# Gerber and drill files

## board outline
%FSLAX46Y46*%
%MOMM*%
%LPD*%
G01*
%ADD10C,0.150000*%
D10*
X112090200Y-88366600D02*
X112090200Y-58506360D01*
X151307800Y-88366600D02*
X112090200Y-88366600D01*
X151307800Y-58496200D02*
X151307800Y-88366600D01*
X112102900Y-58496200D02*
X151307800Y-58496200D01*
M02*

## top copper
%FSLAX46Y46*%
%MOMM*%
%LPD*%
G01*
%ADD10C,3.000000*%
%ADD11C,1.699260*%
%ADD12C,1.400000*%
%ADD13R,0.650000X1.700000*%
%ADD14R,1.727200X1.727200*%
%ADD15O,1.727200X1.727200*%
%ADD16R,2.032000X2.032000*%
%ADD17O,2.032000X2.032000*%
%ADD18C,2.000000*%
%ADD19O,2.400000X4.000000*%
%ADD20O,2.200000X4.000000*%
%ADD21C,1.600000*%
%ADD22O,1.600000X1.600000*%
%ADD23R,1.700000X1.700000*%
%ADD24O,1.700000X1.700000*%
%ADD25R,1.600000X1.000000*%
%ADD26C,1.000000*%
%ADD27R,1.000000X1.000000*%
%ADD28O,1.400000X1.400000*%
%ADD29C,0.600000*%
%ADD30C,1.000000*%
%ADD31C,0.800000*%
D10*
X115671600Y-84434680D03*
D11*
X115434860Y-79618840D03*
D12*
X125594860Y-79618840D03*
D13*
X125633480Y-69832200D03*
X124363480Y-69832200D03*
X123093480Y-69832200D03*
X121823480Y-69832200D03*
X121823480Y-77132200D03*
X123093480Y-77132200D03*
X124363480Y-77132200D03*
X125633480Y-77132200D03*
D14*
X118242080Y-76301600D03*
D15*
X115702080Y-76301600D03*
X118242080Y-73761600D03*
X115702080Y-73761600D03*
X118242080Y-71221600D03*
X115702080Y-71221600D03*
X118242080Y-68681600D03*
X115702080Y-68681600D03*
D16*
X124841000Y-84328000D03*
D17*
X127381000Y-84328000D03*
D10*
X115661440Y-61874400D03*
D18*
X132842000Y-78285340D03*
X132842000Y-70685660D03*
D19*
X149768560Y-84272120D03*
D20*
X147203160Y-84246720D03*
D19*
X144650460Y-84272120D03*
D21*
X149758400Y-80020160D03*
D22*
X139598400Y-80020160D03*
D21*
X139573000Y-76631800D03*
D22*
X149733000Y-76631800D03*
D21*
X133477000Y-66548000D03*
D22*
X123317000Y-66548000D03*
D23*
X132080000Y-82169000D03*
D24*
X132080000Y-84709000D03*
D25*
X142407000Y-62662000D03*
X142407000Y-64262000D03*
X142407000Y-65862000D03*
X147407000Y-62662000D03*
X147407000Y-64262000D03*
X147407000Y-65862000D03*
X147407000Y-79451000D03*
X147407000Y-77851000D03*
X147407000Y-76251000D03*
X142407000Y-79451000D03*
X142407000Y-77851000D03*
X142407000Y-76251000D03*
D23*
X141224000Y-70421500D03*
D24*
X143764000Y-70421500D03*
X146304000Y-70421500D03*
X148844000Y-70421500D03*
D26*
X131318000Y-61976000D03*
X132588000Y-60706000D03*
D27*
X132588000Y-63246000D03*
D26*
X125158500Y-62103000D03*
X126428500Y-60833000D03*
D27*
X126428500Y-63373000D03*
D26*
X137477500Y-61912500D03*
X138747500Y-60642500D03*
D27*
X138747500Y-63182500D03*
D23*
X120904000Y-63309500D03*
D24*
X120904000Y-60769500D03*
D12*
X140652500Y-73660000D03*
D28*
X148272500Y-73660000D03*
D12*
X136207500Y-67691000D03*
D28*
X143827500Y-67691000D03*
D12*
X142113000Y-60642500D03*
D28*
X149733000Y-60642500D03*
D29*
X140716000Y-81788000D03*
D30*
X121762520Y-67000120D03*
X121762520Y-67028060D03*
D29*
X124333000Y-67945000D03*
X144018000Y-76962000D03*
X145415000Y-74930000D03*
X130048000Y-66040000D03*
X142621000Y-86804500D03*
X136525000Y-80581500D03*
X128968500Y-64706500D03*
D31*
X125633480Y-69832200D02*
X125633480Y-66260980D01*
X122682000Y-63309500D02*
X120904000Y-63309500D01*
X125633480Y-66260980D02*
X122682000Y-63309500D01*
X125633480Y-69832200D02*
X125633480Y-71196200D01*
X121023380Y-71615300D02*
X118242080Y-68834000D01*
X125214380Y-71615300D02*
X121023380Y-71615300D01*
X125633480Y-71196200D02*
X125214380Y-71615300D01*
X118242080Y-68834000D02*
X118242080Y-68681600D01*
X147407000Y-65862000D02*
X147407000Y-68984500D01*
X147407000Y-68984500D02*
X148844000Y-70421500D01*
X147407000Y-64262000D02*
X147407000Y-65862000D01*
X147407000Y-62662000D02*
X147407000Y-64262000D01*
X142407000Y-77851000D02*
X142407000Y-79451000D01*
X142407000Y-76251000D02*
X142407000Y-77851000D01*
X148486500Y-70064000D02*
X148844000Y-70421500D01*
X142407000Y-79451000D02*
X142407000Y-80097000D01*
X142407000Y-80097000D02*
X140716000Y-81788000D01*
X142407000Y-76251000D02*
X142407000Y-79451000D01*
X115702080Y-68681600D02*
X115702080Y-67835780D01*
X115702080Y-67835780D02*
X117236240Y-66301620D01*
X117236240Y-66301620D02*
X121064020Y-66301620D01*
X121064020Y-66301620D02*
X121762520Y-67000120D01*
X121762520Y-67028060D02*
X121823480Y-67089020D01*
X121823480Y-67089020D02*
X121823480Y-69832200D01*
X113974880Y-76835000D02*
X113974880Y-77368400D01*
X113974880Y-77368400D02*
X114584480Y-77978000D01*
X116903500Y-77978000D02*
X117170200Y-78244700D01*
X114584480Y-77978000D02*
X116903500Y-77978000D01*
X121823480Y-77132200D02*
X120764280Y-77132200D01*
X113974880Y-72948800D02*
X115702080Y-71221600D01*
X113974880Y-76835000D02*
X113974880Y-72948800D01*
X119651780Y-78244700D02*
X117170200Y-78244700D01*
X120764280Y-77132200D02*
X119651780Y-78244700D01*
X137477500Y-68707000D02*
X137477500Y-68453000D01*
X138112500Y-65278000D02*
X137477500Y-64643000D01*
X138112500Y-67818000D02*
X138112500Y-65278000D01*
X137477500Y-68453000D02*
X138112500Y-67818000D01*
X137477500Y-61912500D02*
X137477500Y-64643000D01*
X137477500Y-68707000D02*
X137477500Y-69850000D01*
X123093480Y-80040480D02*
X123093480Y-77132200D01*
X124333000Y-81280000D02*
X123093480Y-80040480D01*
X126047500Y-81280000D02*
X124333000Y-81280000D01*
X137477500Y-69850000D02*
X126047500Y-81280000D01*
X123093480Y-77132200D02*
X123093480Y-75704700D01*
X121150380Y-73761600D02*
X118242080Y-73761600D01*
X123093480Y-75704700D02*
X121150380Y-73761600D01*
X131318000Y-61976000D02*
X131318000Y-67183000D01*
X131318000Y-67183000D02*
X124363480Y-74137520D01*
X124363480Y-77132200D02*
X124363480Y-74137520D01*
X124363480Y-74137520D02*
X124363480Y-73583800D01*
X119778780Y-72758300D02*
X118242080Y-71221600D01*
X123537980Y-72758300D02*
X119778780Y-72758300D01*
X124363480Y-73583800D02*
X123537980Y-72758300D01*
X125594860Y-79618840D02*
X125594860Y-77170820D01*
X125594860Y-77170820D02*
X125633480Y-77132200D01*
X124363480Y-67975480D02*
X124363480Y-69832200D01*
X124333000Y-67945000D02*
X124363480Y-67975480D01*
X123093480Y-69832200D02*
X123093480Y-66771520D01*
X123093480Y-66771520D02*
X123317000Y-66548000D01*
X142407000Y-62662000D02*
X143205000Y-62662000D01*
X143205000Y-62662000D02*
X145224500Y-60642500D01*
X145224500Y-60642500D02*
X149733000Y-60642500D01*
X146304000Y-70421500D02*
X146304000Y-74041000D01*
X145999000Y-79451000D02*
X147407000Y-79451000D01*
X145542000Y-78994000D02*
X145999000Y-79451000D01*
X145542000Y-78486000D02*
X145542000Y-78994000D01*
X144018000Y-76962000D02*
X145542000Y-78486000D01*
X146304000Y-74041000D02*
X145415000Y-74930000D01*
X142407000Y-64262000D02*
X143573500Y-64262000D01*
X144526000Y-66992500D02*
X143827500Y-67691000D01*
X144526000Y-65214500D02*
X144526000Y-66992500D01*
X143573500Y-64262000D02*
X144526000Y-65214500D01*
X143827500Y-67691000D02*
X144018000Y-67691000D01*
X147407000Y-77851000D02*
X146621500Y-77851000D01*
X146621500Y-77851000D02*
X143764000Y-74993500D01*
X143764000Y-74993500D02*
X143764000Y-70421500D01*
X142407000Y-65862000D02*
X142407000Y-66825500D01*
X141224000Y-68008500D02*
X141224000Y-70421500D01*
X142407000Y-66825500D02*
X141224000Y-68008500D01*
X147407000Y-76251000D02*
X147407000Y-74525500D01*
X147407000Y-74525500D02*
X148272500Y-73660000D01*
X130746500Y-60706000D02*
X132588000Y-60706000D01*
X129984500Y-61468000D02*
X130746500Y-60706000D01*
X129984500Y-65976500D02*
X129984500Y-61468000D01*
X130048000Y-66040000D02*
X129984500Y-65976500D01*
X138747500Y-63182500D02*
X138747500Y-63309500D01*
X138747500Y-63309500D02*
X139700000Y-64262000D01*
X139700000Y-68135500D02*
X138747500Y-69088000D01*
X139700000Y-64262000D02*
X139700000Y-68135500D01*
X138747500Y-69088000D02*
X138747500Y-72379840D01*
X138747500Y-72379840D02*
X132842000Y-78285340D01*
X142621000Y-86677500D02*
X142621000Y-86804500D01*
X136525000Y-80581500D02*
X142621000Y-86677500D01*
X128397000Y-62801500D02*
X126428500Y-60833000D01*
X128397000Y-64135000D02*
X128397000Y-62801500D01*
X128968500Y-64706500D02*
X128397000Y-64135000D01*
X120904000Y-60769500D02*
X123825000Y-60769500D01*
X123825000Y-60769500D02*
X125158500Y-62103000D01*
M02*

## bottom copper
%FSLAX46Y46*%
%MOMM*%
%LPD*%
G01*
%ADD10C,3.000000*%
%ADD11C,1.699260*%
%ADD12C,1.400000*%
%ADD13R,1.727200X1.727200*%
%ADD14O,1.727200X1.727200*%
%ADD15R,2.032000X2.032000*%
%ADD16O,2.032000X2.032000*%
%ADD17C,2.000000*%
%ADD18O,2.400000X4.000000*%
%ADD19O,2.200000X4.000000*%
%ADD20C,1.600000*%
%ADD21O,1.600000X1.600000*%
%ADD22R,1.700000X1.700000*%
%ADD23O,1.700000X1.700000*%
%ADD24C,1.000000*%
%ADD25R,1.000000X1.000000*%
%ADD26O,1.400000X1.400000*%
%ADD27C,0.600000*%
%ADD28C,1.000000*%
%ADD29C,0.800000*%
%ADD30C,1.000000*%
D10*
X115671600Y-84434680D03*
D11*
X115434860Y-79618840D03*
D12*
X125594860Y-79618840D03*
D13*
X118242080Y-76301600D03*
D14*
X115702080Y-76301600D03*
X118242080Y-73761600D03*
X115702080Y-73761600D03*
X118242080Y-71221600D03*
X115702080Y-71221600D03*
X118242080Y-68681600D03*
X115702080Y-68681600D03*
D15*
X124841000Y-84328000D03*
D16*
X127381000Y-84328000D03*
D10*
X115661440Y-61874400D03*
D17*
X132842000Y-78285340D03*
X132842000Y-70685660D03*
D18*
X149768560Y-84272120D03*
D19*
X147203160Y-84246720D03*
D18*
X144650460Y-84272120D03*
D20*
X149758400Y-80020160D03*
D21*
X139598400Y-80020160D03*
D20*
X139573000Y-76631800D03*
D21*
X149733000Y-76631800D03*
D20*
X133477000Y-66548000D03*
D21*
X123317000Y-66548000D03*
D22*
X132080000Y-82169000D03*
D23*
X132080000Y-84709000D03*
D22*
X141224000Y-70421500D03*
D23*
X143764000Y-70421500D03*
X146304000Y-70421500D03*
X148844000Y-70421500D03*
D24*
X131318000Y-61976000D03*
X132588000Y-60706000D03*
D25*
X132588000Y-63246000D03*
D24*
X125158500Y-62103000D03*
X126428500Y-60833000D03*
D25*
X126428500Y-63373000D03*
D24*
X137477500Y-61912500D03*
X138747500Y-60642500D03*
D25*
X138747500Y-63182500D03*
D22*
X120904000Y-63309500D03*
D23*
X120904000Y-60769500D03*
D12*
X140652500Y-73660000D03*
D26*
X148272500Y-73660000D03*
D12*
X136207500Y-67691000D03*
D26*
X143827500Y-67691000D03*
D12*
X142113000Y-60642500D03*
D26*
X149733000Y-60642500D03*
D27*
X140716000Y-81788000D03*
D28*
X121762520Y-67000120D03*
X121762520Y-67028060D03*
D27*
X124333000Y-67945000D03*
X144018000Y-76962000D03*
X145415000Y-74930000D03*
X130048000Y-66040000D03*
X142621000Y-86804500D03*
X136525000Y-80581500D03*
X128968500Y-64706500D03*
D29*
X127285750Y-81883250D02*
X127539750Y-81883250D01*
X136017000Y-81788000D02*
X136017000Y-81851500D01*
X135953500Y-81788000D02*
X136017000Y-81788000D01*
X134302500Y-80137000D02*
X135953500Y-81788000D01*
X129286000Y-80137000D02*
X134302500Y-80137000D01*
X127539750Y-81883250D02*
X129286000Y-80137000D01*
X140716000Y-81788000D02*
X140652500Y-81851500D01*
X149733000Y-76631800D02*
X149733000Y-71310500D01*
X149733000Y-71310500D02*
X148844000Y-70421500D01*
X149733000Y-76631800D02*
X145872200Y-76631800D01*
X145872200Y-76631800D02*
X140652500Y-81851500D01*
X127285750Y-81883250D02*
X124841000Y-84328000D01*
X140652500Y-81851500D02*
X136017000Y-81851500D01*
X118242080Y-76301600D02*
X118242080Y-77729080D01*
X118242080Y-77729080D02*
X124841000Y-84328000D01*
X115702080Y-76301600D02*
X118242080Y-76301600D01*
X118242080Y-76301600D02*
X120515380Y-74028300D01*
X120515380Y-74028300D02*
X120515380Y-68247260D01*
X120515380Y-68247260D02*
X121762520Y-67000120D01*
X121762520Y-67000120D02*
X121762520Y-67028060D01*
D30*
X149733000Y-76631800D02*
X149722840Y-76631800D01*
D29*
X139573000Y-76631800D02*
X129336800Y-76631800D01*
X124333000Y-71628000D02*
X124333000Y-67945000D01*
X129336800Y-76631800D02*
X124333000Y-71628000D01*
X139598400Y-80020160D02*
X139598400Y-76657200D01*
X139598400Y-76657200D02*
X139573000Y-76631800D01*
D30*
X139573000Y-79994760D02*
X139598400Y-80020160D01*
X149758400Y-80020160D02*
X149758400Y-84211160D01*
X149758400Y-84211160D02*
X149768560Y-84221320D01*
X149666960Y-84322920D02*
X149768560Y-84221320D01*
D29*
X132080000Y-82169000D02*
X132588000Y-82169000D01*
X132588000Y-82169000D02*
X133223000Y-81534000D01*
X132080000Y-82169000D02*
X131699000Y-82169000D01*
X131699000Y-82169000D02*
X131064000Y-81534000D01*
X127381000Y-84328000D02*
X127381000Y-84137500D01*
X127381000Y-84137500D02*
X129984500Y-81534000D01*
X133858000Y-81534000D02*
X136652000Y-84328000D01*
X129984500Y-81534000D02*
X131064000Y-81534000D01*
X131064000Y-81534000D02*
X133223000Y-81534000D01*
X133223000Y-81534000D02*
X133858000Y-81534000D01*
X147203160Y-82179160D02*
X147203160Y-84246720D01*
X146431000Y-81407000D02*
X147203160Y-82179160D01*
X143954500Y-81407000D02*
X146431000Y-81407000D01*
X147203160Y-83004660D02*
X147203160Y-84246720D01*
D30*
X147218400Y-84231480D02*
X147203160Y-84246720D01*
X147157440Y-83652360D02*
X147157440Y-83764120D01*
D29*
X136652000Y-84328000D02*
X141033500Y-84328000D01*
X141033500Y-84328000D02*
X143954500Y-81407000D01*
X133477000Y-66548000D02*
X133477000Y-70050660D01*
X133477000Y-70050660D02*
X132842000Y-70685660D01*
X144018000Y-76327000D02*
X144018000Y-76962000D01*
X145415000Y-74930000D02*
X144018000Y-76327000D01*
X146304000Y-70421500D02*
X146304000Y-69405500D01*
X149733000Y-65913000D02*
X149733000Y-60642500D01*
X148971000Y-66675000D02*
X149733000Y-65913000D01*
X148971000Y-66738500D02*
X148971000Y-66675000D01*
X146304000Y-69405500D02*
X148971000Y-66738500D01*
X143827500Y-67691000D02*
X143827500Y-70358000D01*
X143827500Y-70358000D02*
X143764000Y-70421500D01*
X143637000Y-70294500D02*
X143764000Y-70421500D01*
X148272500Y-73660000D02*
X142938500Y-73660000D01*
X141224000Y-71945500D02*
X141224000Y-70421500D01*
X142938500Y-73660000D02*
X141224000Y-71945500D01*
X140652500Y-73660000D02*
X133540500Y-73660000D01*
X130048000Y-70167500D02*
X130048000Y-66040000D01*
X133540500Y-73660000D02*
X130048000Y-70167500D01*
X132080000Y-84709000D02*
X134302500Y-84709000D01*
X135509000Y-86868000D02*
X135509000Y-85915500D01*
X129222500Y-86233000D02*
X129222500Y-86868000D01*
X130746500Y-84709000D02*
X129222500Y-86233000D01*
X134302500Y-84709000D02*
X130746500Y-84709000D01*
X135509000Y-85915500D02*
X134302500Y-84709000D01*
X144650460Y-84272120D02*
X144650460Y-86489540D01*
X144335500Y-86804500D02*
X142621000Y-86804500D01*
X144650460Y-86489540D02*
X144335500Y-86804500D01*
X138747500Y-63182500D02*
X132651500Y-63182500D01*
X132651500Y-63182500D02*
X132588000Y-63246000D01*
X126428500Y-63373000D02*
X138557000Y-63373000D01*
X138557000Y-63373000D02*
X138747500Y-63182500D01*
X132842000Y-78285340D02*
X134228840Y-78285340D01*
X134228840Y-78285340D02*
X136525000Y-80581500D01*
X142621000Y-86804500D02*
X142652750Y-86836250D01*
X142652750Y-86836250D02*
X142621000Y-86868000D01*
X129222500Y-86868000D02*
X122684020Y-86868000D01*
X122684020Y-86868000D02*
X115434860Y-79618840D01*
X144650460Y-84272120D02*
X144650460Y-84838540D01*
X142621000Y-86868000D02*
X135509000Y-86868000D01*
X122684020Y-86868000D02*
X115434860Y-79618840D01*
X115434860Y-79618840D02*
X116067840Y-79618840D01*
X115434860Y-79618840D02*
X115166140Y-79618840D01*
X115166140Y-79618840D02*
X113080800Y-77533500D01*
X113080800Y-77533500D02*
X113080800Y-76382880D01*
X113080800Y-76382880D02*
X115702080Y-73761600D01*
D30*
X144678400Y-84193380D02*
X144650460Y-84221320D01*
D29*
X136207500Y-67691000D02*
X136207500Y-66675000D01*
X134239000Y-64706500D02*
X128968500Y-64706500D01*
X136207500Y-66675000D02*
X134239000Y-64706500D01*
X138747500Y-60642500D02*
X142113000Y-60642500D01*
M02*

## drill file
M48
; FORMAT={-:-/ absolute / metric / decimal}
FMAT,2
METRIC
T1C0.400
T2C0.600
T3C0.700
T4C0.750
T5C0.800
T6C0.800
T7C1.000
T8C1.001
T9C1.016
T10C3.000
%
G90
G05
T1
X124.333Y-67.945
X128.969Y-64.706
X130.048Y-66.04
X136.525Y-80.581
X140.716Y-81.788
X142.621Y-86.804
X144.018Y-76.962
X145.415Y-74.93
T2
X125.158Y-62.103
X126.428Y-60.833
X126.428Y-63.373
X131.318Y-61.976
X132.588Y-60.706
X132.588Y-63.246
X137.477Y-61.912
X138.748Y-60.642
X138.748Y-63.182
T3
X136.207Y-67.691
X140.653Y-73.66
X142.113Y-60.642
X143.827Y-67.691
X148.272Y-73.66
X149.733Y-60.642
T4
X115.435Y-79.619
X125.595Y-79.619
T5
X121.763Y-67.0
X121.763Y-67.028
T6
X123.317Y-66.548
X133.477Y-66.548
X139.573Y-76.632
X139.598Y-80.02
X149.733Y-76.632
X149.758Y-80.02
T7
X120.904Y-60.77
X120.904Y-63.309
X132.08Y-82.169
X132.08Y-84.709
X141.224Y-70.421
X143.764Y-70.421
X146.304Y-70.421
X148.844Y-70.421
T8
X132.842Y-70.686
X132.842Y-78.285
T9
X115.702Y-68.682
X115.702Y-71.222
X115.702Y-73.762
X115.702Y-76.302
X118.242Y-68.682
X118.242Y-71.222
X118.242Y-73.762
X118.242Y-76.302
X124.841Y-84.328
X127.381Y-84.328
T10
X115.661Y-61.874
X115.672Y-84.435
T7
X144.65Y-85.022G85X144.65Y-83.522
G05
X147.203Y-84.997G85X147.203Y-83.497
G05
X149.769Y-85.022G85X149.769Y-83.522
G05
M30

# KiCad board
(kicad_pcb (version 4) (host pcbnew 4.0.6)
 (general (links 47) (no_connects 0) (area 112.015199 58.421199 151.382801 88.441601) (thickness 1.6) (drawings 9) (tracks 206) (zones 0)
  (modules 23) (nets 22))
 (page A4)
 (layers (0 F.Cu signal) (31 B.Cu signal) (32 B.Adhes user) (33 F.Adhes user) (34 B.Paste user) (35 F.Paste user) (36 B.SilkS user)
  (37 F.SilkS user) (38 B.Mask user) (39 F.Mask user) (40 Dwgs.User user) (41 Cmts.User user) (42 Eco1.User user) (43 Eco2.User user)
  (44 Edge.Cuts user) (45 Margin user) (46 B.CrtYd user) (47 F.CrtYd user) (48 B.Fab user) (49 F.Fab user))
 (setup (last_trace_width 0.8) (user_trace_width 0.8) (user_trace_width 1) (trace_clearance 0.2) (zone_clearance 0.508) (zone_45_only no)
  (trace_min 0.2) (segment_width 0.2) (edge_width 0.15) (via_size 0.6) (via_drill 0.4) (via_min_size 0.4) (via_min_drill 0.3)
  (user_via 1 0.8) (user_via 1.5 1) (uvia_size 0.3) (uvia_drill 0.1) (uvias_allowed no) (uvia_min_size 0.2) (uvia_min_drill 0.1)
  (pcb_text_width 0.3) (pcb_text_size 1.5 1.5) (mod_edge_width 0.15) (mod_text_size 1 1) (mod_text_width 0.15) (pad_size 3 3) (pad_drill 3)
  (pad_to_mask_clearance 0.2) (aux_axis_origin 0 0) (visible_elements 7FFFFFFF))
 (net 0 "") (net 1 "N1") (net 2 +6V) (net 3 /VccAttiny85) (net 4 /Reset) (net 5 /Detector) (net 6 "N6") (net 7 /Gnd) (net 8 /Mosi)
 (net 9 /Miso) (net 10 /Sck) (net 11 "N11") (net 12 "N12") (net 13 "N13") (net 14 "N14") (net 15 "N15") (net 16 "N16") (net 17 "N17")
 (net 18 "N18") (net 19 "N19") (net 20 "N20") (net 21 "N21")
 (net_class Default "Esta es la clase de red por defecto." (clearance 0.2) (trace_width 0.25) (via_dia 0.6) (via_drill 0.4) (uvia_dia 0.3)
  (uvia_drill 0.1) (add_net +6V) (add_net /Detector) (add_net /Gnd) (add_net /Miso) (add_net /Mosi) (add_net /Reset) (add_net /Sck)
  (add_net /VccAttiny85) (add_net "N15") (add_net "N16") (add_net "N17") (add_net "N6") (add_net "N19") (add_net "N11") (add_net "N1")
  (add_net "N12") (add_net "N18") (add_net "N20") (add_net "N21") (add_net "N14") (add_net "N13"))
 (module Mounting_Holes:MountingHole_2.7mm (layer F.Cu) (at 115.6716 84.43468)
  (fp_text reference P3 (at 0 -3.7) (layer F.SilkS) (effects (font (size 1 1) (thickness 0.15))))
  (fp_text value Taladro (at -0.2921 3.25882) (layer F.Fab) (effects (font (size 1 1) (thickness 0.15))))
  (pad 1 thru_hole circle (at 0 0) (size 3 3) (drill 3) (layers *.Cu *.Mask) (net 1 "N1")))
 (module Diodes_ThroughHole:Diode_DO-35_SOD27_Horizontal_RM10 (layer F.Cu) (at 125.59538 79.6163 180)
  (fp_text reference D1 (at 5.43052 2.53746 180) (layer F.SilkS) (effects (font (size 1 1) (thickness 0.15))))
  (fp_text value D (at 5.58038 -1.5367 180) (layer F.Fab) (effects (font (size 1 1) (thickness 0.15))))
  (pad 2 thru_hole circle (at 10.16052 -0.00254) (size 1.69926 1.69926) (drill 0.75) (layers *.Cu *.Mask) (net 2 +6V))
  (pad 1 thru_hole circle (at 0.00052 -0.00254) (size 1.4 1.4) (drill 0.75) (layers *.Cu *.Mask) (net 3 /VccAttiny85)))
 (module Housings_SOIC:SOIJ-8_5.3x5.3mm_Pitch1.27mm (layer F.Cu) (at 123.72848 73.4822 270)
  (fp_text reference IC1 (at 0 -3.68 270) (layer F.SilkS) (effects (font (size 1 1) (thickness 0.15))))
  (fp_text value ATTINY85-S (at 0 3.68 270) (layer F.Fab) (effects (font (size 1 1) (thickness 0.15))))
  (pad 1 smd rect (at -3.65 -1.905 270) (size 1.7 0.65) (layers F.Cu F.Paste F.Mask) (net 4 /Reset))
  (pad 2 smd rect (at -3.65 -0.635 270) (size 1.7 0.65) (layers F.Cu F.Paste F.Mask) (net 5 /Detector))
  (pad 3 smd rect (at -3.65 0.635 270) (size 1.7 0.65) (layers F.Cu F.Paste F.Mask) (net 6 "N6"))
  (pad 4 smd rect (at -3.65 1.905 270) (size 1.7 0.65) (layers F.Cu F.Paste F.Mask) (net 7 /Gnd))
  (pad 5 smd rect (at 3.65 1.905 270) (size 1.7 0.65) (layers F.Cu F.Paste F.Mask) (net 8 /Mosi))
  (pad 6 smd rect (at 3.65 0.635 270) (size 1.7 0.65) (layers F.Cu F.Paste F.Mask) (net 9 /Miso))
  (pad 7 smd rect (at 3.65 -0.635 270) (size 1.7 0.65) (layers F.Cu F.Paste F.Mask) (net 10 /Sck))
  (pad 8 smd rect (at 3.65 -1.905 270) (size 1.7 0.65) (layers F.Cu F.Paste F.Mask) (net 3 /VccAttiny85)))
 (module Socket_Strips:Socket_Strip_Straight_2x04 (layer B.Cu) (at 118.24208 76.3016 90)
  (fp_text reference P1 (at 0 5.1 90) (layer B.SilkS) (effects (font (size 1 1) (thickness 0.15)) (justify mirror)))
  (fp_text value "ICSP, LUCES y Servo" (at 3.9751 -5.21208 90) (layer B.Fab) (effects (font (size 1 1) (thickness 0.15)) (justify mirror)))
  (pad 1 thru_hole rect (at 0 0 90) (size 1.7272 1.7272) (drill 1.016) (layers *.Cu *.Mask) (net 7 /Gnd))
  (pad 2 thru_hole oval (at 0 -2.54 90) (size 1.7272 1.7272) (drill 1.016) (layers *.Cu *.Mask) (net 7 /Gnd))
  (pad 3 thru_hole oval (at 2.54 0 90) (size 1.7272 1.7272) (drill 1.016) (layers *.Cu *.Mask) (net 9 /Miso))
  (pad 4 thru_hole oval (at 2.54 -2.54 90) (size 1.7272 1.7272) (drill 1.016) (layers *.Cu *.Mask) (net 2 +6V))
  (pad 5 thru_hole oval (at 5.08 0 90) (size 1.7272 1.7272) (drill 1.016) (layers *.Cu *.Mask) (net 10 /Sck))
  (pad 6 thru_hole oval (at 5.08 -2.54 90) (size 1.7272 1.7272) (drill 1.016) (layers *.Cu *.Mask) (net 8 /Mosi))
  (pad 7 thru_hole oval (at 7.62 0 90) (size 1.7272 1.7272) (drill 1.016) (layers *.Cu *.Mask) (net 4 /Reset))
  (pad 8 thru_hole oval (at 7.62 -2.54 90) (size 1.7272 1.7272) (drill 1.016) (layers *.Cu *.Mask) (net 7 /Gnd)))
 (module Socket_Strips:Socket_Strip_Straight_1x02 (layer F.Cu) (at 124.841 84.328)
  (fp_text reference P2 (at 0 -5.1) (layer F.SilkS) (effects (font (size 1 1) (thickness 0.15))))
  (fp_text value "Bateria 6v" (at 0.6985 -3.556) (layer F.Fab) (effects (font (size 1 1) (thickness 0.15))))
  (pad 1 thru_hole rect (at 0 0) (size 2.032 2.032) (drill 1.016) (layers *.Cu *.Mask) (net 7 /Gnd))
  (pad 2 thru_hole oval (at 2.54 0) (size 2.032 2.032) (drill 1.016) (layers *.Cu *.Mask) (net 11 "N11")))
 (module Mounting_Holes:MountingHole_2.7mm (layer F.Cu) (at 115.66144 61.8744)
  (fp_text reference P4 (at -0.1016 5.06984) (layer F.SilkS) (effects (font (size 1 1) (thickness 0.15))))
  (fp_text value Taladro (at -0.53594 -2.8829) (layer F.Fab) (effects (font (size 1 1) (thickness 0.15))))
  (pad 1 thru_hole circle (at 0 0) (size 3 3) (drill 3) (layers *.Cu *.Mask) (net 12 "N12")))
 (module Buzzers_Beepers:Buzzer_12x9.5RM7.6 (layer F.Cu) (at 132.842 74.4855 90)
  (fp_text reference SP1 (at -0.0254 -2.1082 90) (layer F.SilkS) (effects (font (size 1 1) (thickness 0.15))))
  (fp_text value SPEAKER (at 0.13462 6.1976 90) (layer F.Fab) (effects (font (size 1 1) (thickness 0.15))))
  (pad 1 thru_hole circle (at -3.79984 0 90) (size 2 2) (drill 1.00076) (layers *.Cu *.Mask) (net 2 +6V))
  (pad 2 thru_hole circle (at 3.79984 0 90) (size 2 2) (drill 1.00076) (layers *.Cu *.Mask) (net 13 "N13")))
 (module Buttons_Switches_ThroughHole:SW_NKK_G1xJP (layer B.Cu) (at 147.17776 84.24672 180)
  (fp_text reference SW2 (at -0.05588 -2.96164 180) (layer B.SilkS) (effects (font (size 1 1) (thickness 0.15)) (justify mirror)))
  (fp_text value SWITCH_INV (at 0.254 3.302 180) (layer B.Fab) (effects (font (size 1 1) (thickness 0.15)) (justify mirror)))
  (pad 1 thru_hole oval (at -2.5908 -0.0254 180) (size 2.4 4) (drill oval 1 2.5) (layers *.Cu *.Mask) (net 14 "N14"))
  (pad 2 thru_hole oval (at -0.0254 0 180) (size 2.2 4) (drill oval 1 2.5) (layers *.Cu *.Mask) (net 11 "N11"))
  (pad 3 thru_hole oval (at 2.5273 -0.0254 180) (size 2.4 4) (drill oval 1 2.5) (layers *.Cu *.Mask) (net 2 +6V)))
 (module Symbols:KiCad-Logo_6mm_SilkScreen (layer B.Cu) (at 132.6515 74.676)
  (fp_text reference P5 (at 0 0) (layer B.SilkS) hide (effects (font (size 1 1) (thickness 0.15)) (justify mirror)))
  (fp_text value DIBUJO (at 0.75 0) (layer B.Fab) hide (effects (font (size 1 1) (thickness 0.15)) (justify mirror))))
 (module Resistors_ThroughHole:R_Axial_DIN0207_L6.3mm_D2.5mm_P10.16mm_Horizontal (layer B.Cu) (at 149.7584 80.02016 180)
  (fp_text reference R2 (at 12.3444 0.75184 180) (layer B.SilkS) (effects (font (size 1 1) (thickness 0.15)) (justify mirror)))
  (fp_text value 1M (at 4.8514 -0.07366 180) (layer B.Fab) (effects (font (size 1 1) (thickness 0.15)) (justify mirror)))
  (pad 1 thru_hole circle (at 0 0 180) (size 1.6 1.6) (drill 0.8) (layers *.Cu *.Mask) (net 14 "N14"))
  (pad 2 thru_hole oval (at 10.16 0 180) (size 1.6 1.6) (drill 0.8) (layers *.Cu *.Mask) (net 5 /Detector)))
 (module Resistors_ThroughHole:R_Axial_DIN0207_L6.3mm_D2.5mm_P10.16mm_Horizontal (layer B.Cu) (at 139.573 76.6318)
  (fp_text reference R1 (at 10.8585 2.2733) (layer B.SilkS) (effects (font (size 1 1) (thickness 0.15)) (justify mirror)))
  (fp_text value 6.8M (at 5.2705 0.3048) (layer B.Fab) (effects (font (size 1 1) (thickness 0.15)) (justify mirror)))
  (pad 1 thru_hole circle (at 0 0) (size 1.6 1.6) (drill 0.8) (layers *.Cu *.Mask) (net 5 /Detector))
  (pad 2 thru_hole oval (at 10.16 0) (size 1.6 1.6) (drill 0.8) (layers *.Cu *.Mask) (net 7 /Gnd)))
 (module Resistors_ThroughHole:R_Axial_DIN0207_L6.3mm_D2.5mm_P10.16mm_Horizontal (layer F.Cu) (at 133.477 66.548 180)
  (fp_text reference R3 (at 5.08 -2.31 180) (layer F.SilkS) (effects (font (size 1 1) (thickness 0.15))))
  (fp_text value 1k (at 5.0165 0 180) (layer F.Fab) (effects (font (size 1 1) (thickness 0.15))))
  (pad 1 thru_hole circle (at 0 0 180) (size 1.6 1.6) (drill 0.8) (layers *.Cu *.Mask) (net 13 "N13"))
  (pad 2 thru_hole oval (at 10.16 0 180) (size 1.6 1.6) (drill 0.8) (layers *.Cu *.Mask) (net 6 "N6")))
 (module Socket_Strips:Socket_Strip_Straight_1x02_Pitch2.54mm (layer F.Cu) (at 132.08 82.169)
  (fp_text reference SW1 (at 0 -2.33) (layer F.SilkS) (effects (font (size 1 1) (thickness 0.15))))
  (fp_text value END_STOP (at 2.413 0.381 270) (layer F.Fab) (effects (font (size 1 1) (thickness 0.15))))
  (pad 1 thru_hole rect (at 0 0) (size 1.7 1.7) (drill 1) (layers *.Cu *.Mask) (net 11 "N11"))
  (pad 2 thru_hole oval (at 0 2.54) (size 1.7 1.7) (drill 1) (layers *.Cu *.Mask) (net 2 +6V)))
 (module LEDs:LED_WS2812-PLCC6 (layer F.Cu) (at 144.907 64.262 180)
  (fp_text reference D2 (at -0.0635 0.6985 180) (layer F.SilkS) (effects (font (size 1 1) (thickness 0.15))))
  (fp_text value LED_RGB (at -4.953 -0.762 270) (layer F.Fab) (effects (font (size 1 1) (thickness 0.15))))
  (pad 4 smd rect (at 2.5 1.6 180) (size 1.6 1) (layers F.Cu F.Paste F.Mask) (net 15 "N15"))
  (pad 5 smd rect (at 2.5 0 180) (size 1.6 1) (layers F.Cu F.Paste F.Mask) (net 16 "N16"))
  (pad 6 smd rect (at 2.5 -1.6 180) (size 1.6 1) (layers F.Cu F.Paste F.Mask) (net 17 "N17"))
  (pad 3 smd rect (at -2.5 1.6 180) (size 1.6 1) (layers F.Cu F.Paste F.Mask) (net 7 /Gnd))
  (pad 2 smd rect (at -2.5 0 180) (size 1.6 1) (layers F.Cu F.Paste F.Mask) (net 7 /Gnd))
  (pad 1 smd rect (at -2.5 -1.6 180) (size 1.6 1) (layers F.Cu F.Paste F.Mask) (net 7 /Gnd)))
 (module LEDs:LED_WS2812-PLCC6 (layer F.Cu) (at 144.907 77.851)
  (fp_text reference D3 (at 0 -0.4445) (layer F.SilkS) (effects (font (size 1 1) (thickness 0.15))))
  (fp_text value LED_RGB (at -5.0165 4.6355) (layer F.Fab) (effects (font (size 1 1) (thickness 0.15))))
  (pad 4 smd rect (at 2.5 1.6) (size 1.6 1) (layers F.Cu F.Paste F.Mask) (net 15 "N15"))
  (pad 5 smd rect (at 2.5 0) (size 1.6 1) (layers F.Cu F.Paste F.Mask) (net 16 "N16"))
  (pad 6 smd rect (at 2.5 -1.6) (size 1.6 1) (layers F.Cu F.Paste F.Mask) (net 17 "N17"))
  (pad 3 smd rect (at -2.5 1.6) (size 1.6 1) (layers F.Cu F.Paste F.Mask) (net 7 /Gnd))
  (pad 2 smd rect (at -2.5 0) (size 1.6 1) (layers F.Cu F.Paste F.Mask) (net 7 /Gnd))
  (pad 1 smd rect (at -2.5 -1.6) (size 1.6 1) (layers F.Cu F.Paste F.Mask) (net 7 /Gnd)))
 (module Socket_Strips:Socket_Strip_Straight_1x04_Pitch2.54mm (layer F.Cu) (at 141.224 70.4215 90)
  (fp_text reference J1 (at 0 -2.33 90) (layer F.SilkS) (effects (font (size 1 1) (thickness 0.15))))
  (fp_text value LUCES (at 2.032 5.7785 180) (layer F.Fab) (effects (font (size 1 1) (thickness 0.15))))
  (pad 1 thru_hole rect (at 0 0 90) (size 1.7 1.7) (drill 1) (layers *.Cu *.Mask) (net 17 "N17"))
  (pad 2 thru_hole oval (at 0 2.54 90) (size 1.7 1.7) (drill 1) (layers *.Cu *.Mask) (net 16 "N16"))
  (pad 3 thru_hole oval (at 0 5.08 90) (size 1.7 1.7) (drill 1) (layers *.Cu *.Mask) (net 15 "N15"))
  (pad 4 thru_hole oval (at 0 7.62 90) (size 1.7 1.7) (drill 1) (layers *.Cu *.Mask) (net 7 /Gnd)))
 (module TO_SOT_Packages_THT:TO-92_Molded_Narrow (layer F.Cu) (at 132.588 63.246 90)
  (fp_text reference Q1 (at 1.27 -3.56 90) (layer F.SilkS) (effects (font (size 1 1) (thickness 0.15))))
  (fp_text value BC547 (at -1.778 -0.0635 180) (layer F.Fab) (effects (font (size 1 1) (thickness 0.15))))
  (pad 2 thru_hole circle (at 1.27 -1.27 180) (size 1 1) (drill 0.6) (layers *.Cu *.Mask) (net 10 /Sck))
  (pad 3 thru_hole circle (at 2.54 0 180) (size 1 1) (drill 0.6) (layers *.Cu *.Mask) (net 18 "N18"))
  (pad 1 thru_hole rect (at 0 0 180) (size 1 1) (drill 0.6) (layers *.Cu *.Mask) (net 2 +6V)))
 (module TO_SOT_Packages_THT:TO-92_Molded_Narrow (layer F.Cu) (at 126.4285 63.373 90)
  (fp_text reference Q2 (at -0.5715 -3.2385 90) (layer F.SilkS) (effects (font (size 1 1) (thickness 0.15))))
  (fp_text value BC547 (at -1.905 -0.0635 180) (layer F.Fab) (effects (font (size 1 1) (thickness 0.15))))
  (pad 2 thru_hole circle (at 1.27 -1.27 180) (size 1 1) (drill 0.6) (layers *.Cu *.Mask) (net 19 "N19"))
  (pad 3 thru_hole circle (at 2.54 0 180) (size 1 1) (drill 0.6) (layers *.Cu *.Mask) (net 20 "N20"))
  (pad 1 thru_hole rect (at 0 0 180) (size 1 1) (drill 0.6) (layers *.Cu *.Mask) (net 2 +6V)))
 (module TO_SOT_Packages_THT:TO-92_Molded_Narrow (layer F.Cu) (at 138.7475 63.1825 90)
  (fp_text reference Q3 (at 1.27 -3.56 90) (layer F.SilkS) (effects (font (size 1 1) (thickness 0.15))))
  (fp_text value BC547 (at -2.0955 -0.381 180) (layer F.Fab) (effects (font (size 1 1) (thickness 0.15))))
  (pad 2 thru_hole circle (at 1.27 -1.27 180) (size 1 1) (drill 0.6) (layers *.Cu *.Mask) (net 9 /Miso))
  (pad 3 thru_hole circle (at 2.54 0 180) (size 1 1) (drill 0.6) (layers *.Cu *.Mask) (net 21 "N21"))
  (pad 1 thru_hole rect (at 0 0 180) (size 1 1) (drill 0.6) (layers *.Cu *.Mask) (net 2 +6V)))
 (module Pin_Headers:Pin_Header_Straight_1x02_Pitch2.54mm (layer F.Cu) (at 120.904 63.3095 180)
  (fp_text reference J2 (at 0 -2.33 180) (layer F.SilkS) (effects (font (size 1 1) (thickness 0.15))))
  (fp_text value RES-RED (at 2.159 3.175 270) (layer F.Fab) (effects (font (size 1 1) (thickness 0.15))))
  (pad 1 thru_hole rect (at 0 0 180) (size 1.7 1.7) (drill 1) (layers *.Cu *.Mask) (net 4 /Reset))
  (pad 2 thru_hole oval (at 0 2.54 180) (size 1.7 1.7) (drill 1) (layers *.Cu *.Mask) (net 19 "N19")))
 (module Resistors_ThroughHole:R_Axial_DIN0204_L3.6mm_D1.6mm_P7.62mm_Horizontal (layer F.Cu) (at 140.6525 73.66)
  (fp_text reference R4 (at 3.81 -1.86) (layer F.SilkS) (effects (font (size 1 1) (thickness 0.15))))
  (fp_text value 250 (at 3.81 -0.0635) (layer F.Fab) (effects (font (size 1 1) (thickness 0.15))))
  (pad 1 thru_hole circle (at 0 0) (size 1.4 1.4) (drill 0.7) (layers *.Cu *.Mask) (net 18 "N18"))
  (pad 2 thru_hole oval (at 7.62 0) (size 1.4 1.4) (drill 0.7) (layers *.Cu *.Mask) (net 17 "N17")))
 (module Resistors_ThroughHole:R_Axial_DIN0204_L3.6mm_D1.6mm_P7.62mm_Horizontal (layer F.Cu) (at 136.2075 67.691)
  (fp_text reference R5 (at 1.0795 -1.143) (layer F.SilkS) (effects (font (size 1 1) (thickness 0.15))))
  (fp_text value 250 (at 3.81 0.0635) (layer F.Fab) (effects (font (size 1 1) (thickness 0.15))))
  (pad 1 thru_hole circle (at 0 0) (size 1.4 1.4) (drill 0.7) (layers *.Cu *.Mask) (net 20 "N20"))
  (pad 2 thru_hole oval (at 7.62 0) (size 1.4 1.4) (drill 0.7) (layers *.Cu *.Mask) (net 16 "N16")))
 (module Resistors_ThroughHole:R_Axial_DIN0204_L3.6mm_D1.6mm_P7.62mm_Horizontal (layer F.Cu) (at 142.113 60.6425)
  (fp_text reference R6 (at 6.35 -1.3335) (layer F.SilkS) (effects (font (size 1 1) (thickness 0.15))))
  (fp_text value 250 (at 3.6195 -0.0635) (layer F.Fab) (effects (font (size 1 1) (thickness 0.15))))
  (pad 1 thru_hole circle (at 0 0) (size 1.4 1.4) (drill 0.7) (layers *.Cu *.Mask) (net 21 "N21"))
  (pad 2 thru_hole oval (at 7.62 0) (size 1.4 1.4) (drill 0.7) (layers *.Cu *.Mask) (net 15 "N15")))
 (gr_line (start 112.0902 88.3666) (end 112.0902 58.50636) (angle 90) (layer Edge.Cuts) (width 0.15))
 (gr_line (start 151.3078 88.3666) (end 112.0902 88.3666) (angle 90) (layer Edge.Cuts) (width 0.15))
 (gr_line (start 151.3078 58.4962) (end 151.3078 88.3666) (angle 90) (layer Edge.Cuts) (width 0.15))
 (gr_line (start 112.1029 58.4962) (end 151.3078 58.4962) (angle 90) (layer Edge.Cuts) (width 0.15))
 (segment (start 125.63348 69.8322) (end 125.63348 66.26098) (width 0.8) (layer F.Cu) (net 4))
 (segment (start 122.682 63.3095) (end 120.904 63.3095) (width 0.8) (layer F.Cu) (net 4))
 (segment (start 125.63348 66.26098) (end 122.682 63.3095) (width 0.8) (layer F.Cu) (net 4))
 (segment (start 125.63348 69.8322) (end 125.63348 71.1962) (width 0.8) (layer F.Cu) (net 4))
 (segment (start 121.02338 71.6153) (end 118.24208 68.834) (width 0.8) (layer F.Cu) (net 4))
 (segment (start 125.21438 71.6153) (end 121.02338 71.6153) (width 0.8) (layer F.Cu) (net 4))
 (segment (start 125.63348 71.1962) (end 125.21438 71.6153) (width 0.8) (layer F.Cu) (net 4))
 (segment (start 118.24208 68.834) (end 118.24208 68.6816) (width 0.8) (layer F.Cu) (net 4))
 (segment (start 127.28575 81.88325) (end 127.53975 81.88325) (width 0.8) (layer B.Cu) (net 7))
 (segment (start 136.017 81.788) (end 136.017 81.8515) (width 0.8) (layer B.Cu) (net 7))
 (segment (start 135.9535 81.788) (end 136.017 81.788) (width 0.8) (layer B.Cu) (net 7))
 (segment (start 134.3025 80.137) (end 135.9535 81.788) (width 0.8) (layer B.Cu) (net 7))
 (segment (start 129.286 80.137) (end 134.3025 80.137) (width 0.8) (layer B.Cu) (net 7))
 (segment (start 127.53975 81.88325) (end 129.286 80.137) (width 0.8) (layer B.Cu) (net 7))
 (segment (start 147.407 65.862) (end 147.407 68.9845) (width 0.8) (layer F.Cu) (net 7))
 (segment (start 147.407 68.9845) (end 148.844 70.4215) (width 0.8) (layer F.Cu) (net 7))
 (segment (start 147.407 64.262) (end 147.407 65.862) (width 0.8) (layer F.Cu) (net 7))
 (segment (start 147.407 62.662) (end 147.407 64.262) (width 0.8) (layer F.Cu) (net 7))
 (segment (start 142.407 77.851) (end 142.407 79.451) (width 0.8) (layer F.Cu) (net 7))
 (segment (start 142.407 76.251) (end 142.407 77.851) (width 0.8) (layer F.Cu) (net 7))
 (segment (start 148.4865 70.064) (end 148.844 70.4215) (width 0.8) (layer F.Cu) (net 7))
 (segment (start 142.407 79.451) (end 142.407 80.097) (width 0.8) (layer F.Cu) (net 7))
 (segment (start 142.407 80.097) (end 140.716 81.788) (width 0.8) (layer F.Cu) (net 7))
 (via (at 140.716 81.788) (size 0.6) (drill 0.4) (layers F.Cu B.Cu) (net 7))
 (segment (start 140.716 81.788) (end 140.6525 81.8515) (width 0.8) (layer B.Cu) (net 7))
 (segment (start 142.407 76.251) (end 142.407 79.451) (width 0.8) (layer F.Cu) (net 7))
 (segment (start 149.733 76.6318) (end 149.733 71.3105) (width 0.8) (layer B.Cu) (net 7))
 (segment (start 149.733 71.3105) (end 148.844 70.4215) (width 0.8) (layer B.Cu) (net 7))
 (segment (start 149.733 76.6318) (end 145.8722 76.6318) (width 0.8) (layer B.Cu) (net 7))
 (segment (start 145.8722 76.6318) (end 140.6525 81.8515) (width 0.8) (layer B.Cu) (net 7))
 (segment (start 127.28575 81.88325) (end 124.841 84.328) (width 0.8) (layer B.Cu) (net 7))
 (segment (start 140.6525 81.8515) (end 136.017 81.8515) (width 0.8) (layer B.Cu) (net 7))
 (segment (start 118.24208 76.3016) (end 118.24208 77.72908) (width 0.8) (layer B.Cu) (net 7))
 (segment (start 118.24208 77.72908) (end 124.841 84.328) (width 0.8) (layer B.Cu) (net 7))
 (segment (start 115.70208 76.3016) (end 118.24208 76.3016) (width 0.8) (layer B.Cu) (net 7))
 (segment (start 118.24208 76.3016) (end 120.51538 74.0283) (width 0.8) (layer B.Cu) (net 7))
 (segment (start 120.51538 74.0283) (end 120.51538 68.24726) (width 0.8) (layer B.Cu) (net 7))
 (segment (start 120.51538 68.24726) (end 121.76252 67.00012) (width 0.8) (layer B.Cu) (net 7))
 (segment (start 115.70208 68.6816) (end 115.70208 67.83578) (width 0.8) (layer F.Cu) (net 7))
 (segment (start 115.70208 67.83578) (end 117.23624 66.30162) (width 0.8) (layer F.Cu) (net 7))
 (segment (start 117.23624 66.30162) (end 121.06402 66.30162) (width 0.8) (layer F.Cu) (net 7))
 (segment (start 121.06402 66.30162) (end 121.76252 67.00012) (width 0.8) (layer F.Cu) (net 7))
 (via (at 121.76252 67.00012) (size 1) (drill 0.8) (layers F.Cu B.Cu) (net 7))
 (segment (start 121.76252 67.00012) (end 121.76252 67.02806) (width 0.8) (layer B.Cu) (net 7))
 (via (at 121.76252 67.02806) (size 1) (drill 0.8) (layers F.Cu B.Cu) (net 7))
 (segment (start 121.76252 67.02806) (end 121.82348 67.08902) (width 0.8) (layer F.Cu) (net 7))
 (segment (start 121.82348 67.08902) (end 121.82348 69.8322) (width 0.8) (layer F.Cu) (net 7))
 (segment (start 149.733 76.6318) (end 149.72284 76.6318) (width 1) (layer B.Cu) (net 7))
 (segment (start 113.97488 76.835) (end 113.97488 77.3684) (width 0.8) (layer F.Cu) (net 8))
 (segment (start 113.97488 77.3684) (end 114.58448 77.978) (width 0.8) (layer F.Cu) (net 8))
 (segment (start 116.9035 77.978) (end 117.1702 78.2447) (width 0.8) (layer F.Cu) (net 8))
 (segment (start 114.58448 77.978) (end 116.9035 77.978) (width 0.8) (layer F.Cu) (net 8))
 (segment (start 121.82348 77.1322) (end 120.76428 77.1322) (width 0.8) (layer F.Cu) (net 8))
 (segment (start 113.97488 72.9488) (end 115.70208 71.2216) (width 0.8) (layer F.Cu) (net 8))
 (segment (start 113.97488 76.835) (end 113.97488 72.9488) (width 0.8) (layer F.Cu) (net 8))
 (segment (start 119.65178 78.2447) (end 117.1702 78.2447) (width 0.8) (layer F.Cu) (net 8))
 (segment (start 120.76428 77.1322) (end 119.65178 78.2447) (width 0.8) (layer F.Cu) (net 8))
 (segment (start 137.4775 68.707) (end 137.4775 68.453) (width 0.8) (layer F.Cu) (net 9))
 (segment (start 138.1125 65.278) (end 137.4775 64.643) (width 0.8) (layer F.Cu) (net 9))
 (segment (start 138.1125 67.818) (end 138.1125 65.278) (width 0.8) (layer F.Cu) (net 9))
 (segment (start 137.4775 68.453) (end 138.1125 67.818) (width 0.8) (layer F.Cu) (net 9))
 (segment (start 137.4775 61.9125) (end 137.4775 64.643) (width 0.8) (layer F.Cu) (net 9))
 (segment (start 137.4775 68.707) (end 137.4775 69.85) (width 0.8) (layer F.Cu) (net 9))
 (segment (start 123.09348 80.04048) (end 123.09348 77.1322) (width 0.8) (layer F.Cu) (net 9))
 (segment (start 124.333 81.28) (end 123.09348 80.04048) (width 0.8) (layer F.Cu) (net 9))
 (segment (start 126.0475 81.28) (end 124.333 81.28) (width 0.8) (layer F.Cu) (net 9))
 (segment (start 137.4775 69.85) (end 126.0475 81.28) (width 0.8) (layer F.Cu) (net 9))
 (segment (start 123.09348 77.1322) (end 123.09348 75.7047) (width 0.8) (layer F.Cu) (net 9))
 (segment (start 121.15038 73.7616) (end 118.24208 73.7616) (width 0.8) (layer F.Cu) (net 9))
 (segment (start 123.09348 75.7047) (end 121.15038 73.7616) (width 0.8) (layer F.Cu) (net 9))
 (segment (start 131.318 61.976) (end 131.318 67.183) (width 0.8) (layer F.Cu) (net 10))
 (segment (start 131.318 67.183) (end 124.36348 74.13752) (width 0.8) (layer F.Cu) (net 10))
 (segment (start 124.36348 77.1322) (end 124.36348 74.13752) (width 0.8) (layer F.Cu) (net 10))
 (segment (start 124.36348 74.13752) (end 124.36348 73.5838) (width 0.8) (layer F.Cu) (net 10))
 (segment (start 119.77878 72.7583) (end 118.24208 71.2216) (width 0.8) (layer F.Cu) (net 10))
 (segment (start 123.53798 72.7583) (end 119.77878 72.7583) (width 0.8) (layer F.Cu) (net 10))
 (segment (start 124.36348 73.5838) (end 123.53798 72.7583) (width 0.8) (layer F.Cu) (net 10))
 (segment (start 125.59486 79.61884) (end 125.59486 77.17082) (width 0.8) (layer F.Cu) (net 3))
 (segment (start 125.59486 77.17082) (end 125.63348 77.1322) (width 0.8) (layer F.Cu) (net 3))
 (segment (start 139.573 76.6318) (end 129.3368 76.6318) (width 0.8) (layer B.Cu) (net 5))
 (segment (start 124.36348 67.97548) (end 124.36348 69.8322) (width 0.8) (layer F.Cu) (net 5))
 (segment (start 124.333 67.945) (end 124.36348 67.97548) (width 0.8) (layer F.Cu) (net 5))
 (via (at 124.333 67.945) (size 0.6) (drill 0.4) (layers F.Cu B.Cu) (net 5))
 (segment (start 124.333 71.628) (end 124.333 67.945) (width 0.8) (layer B.Cu) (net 5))
 (segment (start 129.3368 76.6318) (end 124.333 71.628) (width 0.8) (layer B.Cu) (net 5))
 (segment (start 139.5984 80.02016) (end 139.5984 76.6572) (width 0.8) (layer B.Cu) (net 5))
 (segment (start 139.5984 76.6572) (end 139.573 76.6318) (width 0.8) (layer B.Cu) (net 5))
 (segment (start 139.573 79.99476) (end 139.5984 80.02016) (width 1) (layer B.Cu) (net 5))
 (segment (start 149.7584 80.02016) (end 149.7584 84.21116) (width 1) (layer B.Cu) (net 14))
 (segment (start 149.7584 84.21116) (end 149.76856 84.22132) (width 1) (layer B.Cu) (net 14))
 (segment (start 149.66696 84.32292) (end 149.76856 84.22132) (width 1) (layer B.Cu) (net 14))
 (segment (start 123.09348 69.8322) (end 123.09348 66.77152) (width 0.8) (layer F.Cu) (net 6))
 (segment (start 123.09348 66.77152) (end 123.317 66.548) (width 0.8) (layer F.Cu) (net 6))
 (segment (start 132.08 82.169) (end 132.588 82.169) (width 0.8) (layer B.Cu) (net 11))
 (segment (start 132.588 82.169) (end 133.223 81.534) (width 0.8) (layer B.Cu) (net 11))
 (segment (start 132.08 82.169) (end 131.699 82.169) (width 0.8) (layer B.Cu) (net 11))
 (segment (start 131.699 82.169) (end 131.064 81.534) (width 0.8) (layer B.Cu) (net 11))
 (segment (start 127.381 84.328) (end 127.381 84.1375) (width 0.8) (layer B.Cu) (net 11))
 (segment (start 127.381 84.1375) (end 129.9845 81.534) (width 0.8) (layer B.Cu) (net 11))
 (segment (start 133.858 81.534) (end 136.652 84.328) (width 0.8) (layer B.Cu) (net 11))
 (segment (start 129.9845 81.534) (end 131.064 81.534) (width 0.8) (layer B.Cu) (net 11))
 (segment (start 131.064 81.534) (end 133.223 81.534) (width 0.8) (layer B.Cu) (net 11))
 (segment (start 133.223 81.534) (end 133.858 81.534) (width 0.8) (layer B.Cu) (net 11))
 (segment (start 147.20316 82.17916) (end 147.20316 84.24672) (width 0.8) (layer B.Cu) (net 11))
 (segment (start 146.431 81.407) (end 147.20316 82.17916) (width 0.8) (layer B.Cu) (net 11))
 (segment (start 143.9545 81.407) (end 146.431 81.407) (width 0.8) (layer B.Cu) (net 11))
 (segment (start 147.20316 83.00466) (end 147.20316 84.24672) (width 0.8) (layer B.Cu) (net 11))
 (segment (start 147.2184 84.23148) (end 147.20316 84.24672) (width 1) (layer B.Cu) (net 11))
 (segment (start 147.15744 83.65236) (end 147.15744 83.76412) (width 1) (layer B.Cu) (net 11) (status 30))
 (segment (start 136.652 84.328) (end 141.0335 84.328) (width 0.8) (layer B.Cu) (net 11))
 (segment (start 141.0335 84.328) (end 143.9545 81.407) (width 0.8) (layer B.Cu) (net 11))
 (segment (start 133.477 66.548) (end 133.477 70.05066) (width 0.8) (layer B.Cu) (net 13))
 (segment (start 133.477 70.05066) (end 132.842 70.68566) (width 0.8) (layer B.Cu) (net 13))
 (segment (start 142.407 62.662) (end 143.205 62.662) (width 0.8) (layer F.Cu) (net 15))
 (segment (start 143.205 62.662) (end 145.2245 60.6425) (width 0.8) (layer F.Cu) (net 15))
 (segment (start 145.2245 60.6425) (end 149.733 60.6425) (width 0.8) (layer F.Cu) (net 15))
 (segment (start 146.304 70.4215) (end 146.304 74.041) (width 0.8) (layer F.Cu) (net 15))
 (segment (start 145.999 79.451) (end 147.407 79.451) (width 0.8) (layer F.Cu) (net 15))
 (segment (start 145.542 78.994) (end 145.999 79.451) (width 0.8) (layer F.Cu) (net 15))
 (segment (start 145.542 78.486) (end 145.542 78.994) (width 0.8) (layer F.Cu) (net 15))
 (segment (start 144.018 76.962) (end 145.542 78.486) (width 0.8) (layer F.Cu) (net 15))
 (via (at 144.018 76.962) (size 0.6) (drill 0.4) (layers F.Cu B.Cu) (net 15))
 (segment (start 144.018 76.327) (end 144.018 76.962) (width 0.8) (layer B.Cu) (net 15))
 (segment (start 145.415 74.93) (end 144.018 76.327) (width 0.8) (layer B.Cu) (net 15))
 (via (at 145.415 74.93) (size 0.6) (drill 0.4) (layers F.Cu B.Cu) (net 15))
 (segment (start 146.304 74.041) (end 145.415 74.93) (width 0.8) (layer F.Cu) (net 15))
 (segment (start 146.304 70.4215) (end 146.304 69.4055) (width 0.8) (layer B.Cu) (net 15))
 (segment (start 149.733 65.913) (end 149.733 60.6425) (width 0.8) (layer B.Cu) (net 15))
 (segment (start 148.971 66.675) (end 149.733 65.913) (width 0.8) (layer B.Cu) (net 15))
 (segment (start 148.971 66.7385) (end 148.971 66.675) (width 0.8) (layer B.Cu) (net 15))
 (segment (start 146.304 69.4055) (end 148.971 66.7385) (width 0.8) (layer B.Cu) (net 15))
 (segment (start 142.407 64.262) (end 143.5735 64.262) (width 0.8) (layer F.Cu) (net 16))
 (segment (start 144.526 66.9925) (end 143.8275 67.691) (width 0.8) (layer F.Cu) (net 16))
 (segment (start 144.526 65.2145) (end 144.526 66.9925) (width 0.8) (layer F.Cu) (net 16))
 (segment (start 143.5735 64.262) (end 144.526 65.2145) (width 0.8) (layer F.Cu) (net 16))
 (segment (start 143.8275 67.691) (end 144.018 67.691) (width 0.8) (layer F.Cu) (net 16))
 (segment (start 147.407 77.851) (end 146.6215 77.851) (width 0.8) (layer F.Cu) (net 16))
 (segment (start 146.6215 77.851) (end 143.764 74.9935) (width 0.8) (layer F.Cu) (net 16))
 (segment (start 143.764 74.9935) (end 143.764 70.4215) (width 0.8) (layer F.Cu) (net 16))
 (segment (start 143.8275 67.691) (end 143.8275 70.358) (width 0.8) (layer B.Cu) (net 16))
 (segment (start 143.8275 70.358) (end 143.764 70.4215) (width 0.8) (layer B.Cu) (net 16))
 (segment (start 143.637 70.2945) (end 143.764 70.4215) (width 0.8) (layer B.Cu) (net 16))
 (segment (start 142.407 65.862) (end 142.407 66.8255) (width 0.8) (layer F.Cu) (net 17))
 (segment (start 141.224 68.0085) (end 141.224 70.4215) (width 0.8) (layer F.Cu) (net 17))
 (segment (start 142.407 66.8255) (end 141.224 68.0085) (width 0.8) (layer F.Cu) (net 17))
 (segment (start 147.407 76.251) (end 147.407 74.5255) (width 0.8) (layer F.Cu) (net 17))
 (segment (start 147.407 74.5255) (end 148.2725 73.66) (width 0.8) (layer F.Cu) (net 17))
 (segment (start 148.2725 73.66) (end 142.9385 73.66) (width 0.8) (layer B.Cu) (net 17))
 (segment (start 141.224 71.9455) (end 141.224 70.4215) (width 0.8) (layer B.Cu) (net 17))
 (segment (start 142.9385 73.66) (end 141.224 71.9455) (width 0.8) (layer B.Cu) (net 17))
 (segment (start 140.6525 73.66) (end 133.5405 73.66) (width 0.8) (layer B.Cu) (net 18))
 (segment (start 130.7465 60.706) (end 132.588 60.706) (width 0.8) (layer F.Cu) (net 18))
 (segment (start 129.9845 61.468) (end 130.7465 60.706) (width 0.8) (layer F.Cu) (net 18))
 (segment (start 129.9845 65.9765) (end 129.9845 61.468) (width 0.8) (layer F.Cu) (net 18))
 (segment (start 130.048 66.04) (end 129.9845 65.9765) (width 0.8) (layer F.Cu) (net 18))
 (via (at 130.048 66.04) (size 0.6) (drill 0.4) (layers F.Cu B.Cu) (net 18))
 (segment (start 130.048 70.1675) (end 130.048 66.04) (width 0.8) (layer B.Cu) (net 18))
 (segment (start 133.5405 73.66) (end 130.048 70.1675) (width 0.8) (layer B.Cu) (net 18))
 (segment (start 132.08 84.709) (end 134.3025 84.709) (width 0.8) (layer B.Cu) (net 2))
 (segment (start 135.509 86.868) (end 135.509 85.9155) (width 0.8) (layer B.Cu) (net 2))
 (segment (start 129.2225 86.233) (end 129.2225 86.868) (width 0.8) (layer B.Cu) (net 2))
 (segment (start 130.7465 84.709) (end 129.2225 86.233) (width 0.8) (layer B.Cu) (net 2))
 (segment (start 134.3025 84.709) (end 130.7465 84.709) (width 0.8) (layer B.Cu) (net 2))
 (segment (start 135.509 85.9155) (end 134.3025 84.709) (width 0.8) (layer B.Cu) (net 2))
 (segment (start 144.65046 84.27212) (end 144.65046 86.48954) (width 0.8) (layer B.Cu) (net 2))
 (segment (start 144.3355 86.8045) (end 142.621 86.8045) (width 0.8) (layer B.Cu) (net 2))
 (segment (start 144.65046 86.48954) (end 144.3355 86.8045) (width 0.8) (layer B.Cu) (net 2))
 (segment (start 138.7475 63.1825) (end 138.7475 63.3095) (width 0.8) (layer F.Cu) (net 2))
 (segment (start 138.7475 63.3095) (end 139.7 64.262) (width 0.8) (layer F.Cu) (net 2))
 (segment (start 139.7 68.1355) (end 138.7475 69.088) (width 0.8) (layer F.Cu) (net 2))
 (segment (start 139.7 64.262) (end 139.7 68.1355) (width 0.8) (layer F.Cu) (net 2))
 (segment (start 138.7475 63.1825) (end 132.6515 63.1825) (width 0.8) (layer B.Cu) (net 2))
 (segment (start 132.6515 63.1825) (end 132.588 63.246) (width 0.8) (layer B.Cu) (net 2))
 (segment (start 138.7475 69.088) (end 138.7475 72.37984) (width 0.8) (layer F.Cu) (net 2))
 (segment (start 138.7475 72.37984) (end 132.842 78.28534) (width 0.8) (layer F.Cu) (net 2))
 (segment (start 126.4285 63.373) (end 138.557 63.373) (width 0.8) (layer B.Cu) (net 2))
 (segment (start 138.557 63.373) (end 138.7475 63.1825) (width 0.8) (layer B.Cu) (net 2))
 (segment (start 132.842 78.28534) (end 134.22884 78.28534) (width 0.8) (layer B.Cu) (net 2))
 (via (at 142.621 86.8045) (size 0.6) (drill 0.4) (layers F.Cu B.Cu) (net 2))
 (segment (start 142.621 86.6775) (end 142.621 86.8045) (width 0.8) (layer F.Cu) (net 2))
 (segment (start 136.525 80.5815) (end 142.621 86.6775) (width 0.8) (layer F.Cu) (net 2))
 (via (at 136.525 80.5815) (size 0.6) (drill 0.4) (layers F.Cu B.Cu) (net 2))
 (segment (start 134.22884 78.28534) (end 136.525 80.5815) (width 0.8) (layer B.Cu) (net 2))
 (segment (start 142.621 86.8045) (end 142.65275 86.83625) (width 0.8) (layer B.Cu) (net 2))
 (segment (start 142.65275 86.83625) (end 142.621 86.868) (width 0.8) (layer B.Cu) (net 2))
 (segment (start 129.2225 86.868) (end 122.68402 86.868) (width 0.8) (layer B.Cu) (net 2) (status 10))
 (segment (start 122.68402 86.868) (end 115.43486 79.61884) (width 0.8) (layer B.Cu) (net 2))
 (segment (start 144.65046 84.27212) (end 144.65046 84.83854) (width 0.8) (layer B.Cu) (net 2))
 (segment (start 142.621 86.868) (end 135.509 86.868) (width 0.8) (layer B.Cu) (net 2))
 (segment (start 122.68402 86.868) (end 115.43486 79.61884) (width 0.8) (layer B.Cu) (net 2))
 (segment (start 115.43486 79.61884) (end 116.06784 79.61884) (width 0.8) (layer B.Cu) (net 2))
 (segment (start 115.43486 79.61884) (end 115.16614 79.61884) (width 0.8) (layer B.Cu) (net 2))
 (segment (start 115.16614 79.61884) (end 113.0808 77.5335) (width 0.8) (layer B.Cu) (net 2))
 (segment (start 113.0808 77.5335) (end 113.0808 76.38288) (width 0.8) (layer B.Cu) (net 2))
 (segment (start 113.0808 76.38288) (end 115.70208 73.7616) (width 0.8) (layer B.Cu) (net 2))
 (segment (start 144.6784 84.19338) (end 144.65046 84.22132) (width 1) (layer B.Cu) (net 2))
 (segment (start 136.2075 67.691) (end 136.2075 66.675) (width 0.8) (layer B.Cu) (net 20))
 (segment (start 128.397 62.8015) (end 126.4285 60.833) (width 0.8) (layer F.Cu) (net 20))
 (segment (start 128.397 64.135) (end 128.397 62.8015) (width 0.8) (layer F.Cu) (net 20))
 (segment (start 128.9685 64.7065) (end 128.397 64.135) (width 0.8) (layer F.Cu) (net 20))
 (via (at 128.9685 64.7065) (size 0.6) (drill 0.4) (layers F.Cu B.Cu) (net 20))
 (segment (start 134.239 64.7065) (end 128.9685 64.7065) (width 0.8) (layer B.Cu) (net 20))
 (segment (start 136.2075 66.675) (end 134.239 64.7065) (width 0.8) (layer B.Cu) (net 20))
 (segment (start 138.7475 60.6425) (end 142.113 60.6425) (width 0.8) (layer B.Cu) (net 21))
 (segment (start 120.904 60.7695) (end 123.825 60.7695) (width 0.8) (layer F.Cu) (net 19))
 (segment (start 123.825 60.7695) (end 125.1585 62.103) (width 0.8) (layer F.Cu) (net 19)))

